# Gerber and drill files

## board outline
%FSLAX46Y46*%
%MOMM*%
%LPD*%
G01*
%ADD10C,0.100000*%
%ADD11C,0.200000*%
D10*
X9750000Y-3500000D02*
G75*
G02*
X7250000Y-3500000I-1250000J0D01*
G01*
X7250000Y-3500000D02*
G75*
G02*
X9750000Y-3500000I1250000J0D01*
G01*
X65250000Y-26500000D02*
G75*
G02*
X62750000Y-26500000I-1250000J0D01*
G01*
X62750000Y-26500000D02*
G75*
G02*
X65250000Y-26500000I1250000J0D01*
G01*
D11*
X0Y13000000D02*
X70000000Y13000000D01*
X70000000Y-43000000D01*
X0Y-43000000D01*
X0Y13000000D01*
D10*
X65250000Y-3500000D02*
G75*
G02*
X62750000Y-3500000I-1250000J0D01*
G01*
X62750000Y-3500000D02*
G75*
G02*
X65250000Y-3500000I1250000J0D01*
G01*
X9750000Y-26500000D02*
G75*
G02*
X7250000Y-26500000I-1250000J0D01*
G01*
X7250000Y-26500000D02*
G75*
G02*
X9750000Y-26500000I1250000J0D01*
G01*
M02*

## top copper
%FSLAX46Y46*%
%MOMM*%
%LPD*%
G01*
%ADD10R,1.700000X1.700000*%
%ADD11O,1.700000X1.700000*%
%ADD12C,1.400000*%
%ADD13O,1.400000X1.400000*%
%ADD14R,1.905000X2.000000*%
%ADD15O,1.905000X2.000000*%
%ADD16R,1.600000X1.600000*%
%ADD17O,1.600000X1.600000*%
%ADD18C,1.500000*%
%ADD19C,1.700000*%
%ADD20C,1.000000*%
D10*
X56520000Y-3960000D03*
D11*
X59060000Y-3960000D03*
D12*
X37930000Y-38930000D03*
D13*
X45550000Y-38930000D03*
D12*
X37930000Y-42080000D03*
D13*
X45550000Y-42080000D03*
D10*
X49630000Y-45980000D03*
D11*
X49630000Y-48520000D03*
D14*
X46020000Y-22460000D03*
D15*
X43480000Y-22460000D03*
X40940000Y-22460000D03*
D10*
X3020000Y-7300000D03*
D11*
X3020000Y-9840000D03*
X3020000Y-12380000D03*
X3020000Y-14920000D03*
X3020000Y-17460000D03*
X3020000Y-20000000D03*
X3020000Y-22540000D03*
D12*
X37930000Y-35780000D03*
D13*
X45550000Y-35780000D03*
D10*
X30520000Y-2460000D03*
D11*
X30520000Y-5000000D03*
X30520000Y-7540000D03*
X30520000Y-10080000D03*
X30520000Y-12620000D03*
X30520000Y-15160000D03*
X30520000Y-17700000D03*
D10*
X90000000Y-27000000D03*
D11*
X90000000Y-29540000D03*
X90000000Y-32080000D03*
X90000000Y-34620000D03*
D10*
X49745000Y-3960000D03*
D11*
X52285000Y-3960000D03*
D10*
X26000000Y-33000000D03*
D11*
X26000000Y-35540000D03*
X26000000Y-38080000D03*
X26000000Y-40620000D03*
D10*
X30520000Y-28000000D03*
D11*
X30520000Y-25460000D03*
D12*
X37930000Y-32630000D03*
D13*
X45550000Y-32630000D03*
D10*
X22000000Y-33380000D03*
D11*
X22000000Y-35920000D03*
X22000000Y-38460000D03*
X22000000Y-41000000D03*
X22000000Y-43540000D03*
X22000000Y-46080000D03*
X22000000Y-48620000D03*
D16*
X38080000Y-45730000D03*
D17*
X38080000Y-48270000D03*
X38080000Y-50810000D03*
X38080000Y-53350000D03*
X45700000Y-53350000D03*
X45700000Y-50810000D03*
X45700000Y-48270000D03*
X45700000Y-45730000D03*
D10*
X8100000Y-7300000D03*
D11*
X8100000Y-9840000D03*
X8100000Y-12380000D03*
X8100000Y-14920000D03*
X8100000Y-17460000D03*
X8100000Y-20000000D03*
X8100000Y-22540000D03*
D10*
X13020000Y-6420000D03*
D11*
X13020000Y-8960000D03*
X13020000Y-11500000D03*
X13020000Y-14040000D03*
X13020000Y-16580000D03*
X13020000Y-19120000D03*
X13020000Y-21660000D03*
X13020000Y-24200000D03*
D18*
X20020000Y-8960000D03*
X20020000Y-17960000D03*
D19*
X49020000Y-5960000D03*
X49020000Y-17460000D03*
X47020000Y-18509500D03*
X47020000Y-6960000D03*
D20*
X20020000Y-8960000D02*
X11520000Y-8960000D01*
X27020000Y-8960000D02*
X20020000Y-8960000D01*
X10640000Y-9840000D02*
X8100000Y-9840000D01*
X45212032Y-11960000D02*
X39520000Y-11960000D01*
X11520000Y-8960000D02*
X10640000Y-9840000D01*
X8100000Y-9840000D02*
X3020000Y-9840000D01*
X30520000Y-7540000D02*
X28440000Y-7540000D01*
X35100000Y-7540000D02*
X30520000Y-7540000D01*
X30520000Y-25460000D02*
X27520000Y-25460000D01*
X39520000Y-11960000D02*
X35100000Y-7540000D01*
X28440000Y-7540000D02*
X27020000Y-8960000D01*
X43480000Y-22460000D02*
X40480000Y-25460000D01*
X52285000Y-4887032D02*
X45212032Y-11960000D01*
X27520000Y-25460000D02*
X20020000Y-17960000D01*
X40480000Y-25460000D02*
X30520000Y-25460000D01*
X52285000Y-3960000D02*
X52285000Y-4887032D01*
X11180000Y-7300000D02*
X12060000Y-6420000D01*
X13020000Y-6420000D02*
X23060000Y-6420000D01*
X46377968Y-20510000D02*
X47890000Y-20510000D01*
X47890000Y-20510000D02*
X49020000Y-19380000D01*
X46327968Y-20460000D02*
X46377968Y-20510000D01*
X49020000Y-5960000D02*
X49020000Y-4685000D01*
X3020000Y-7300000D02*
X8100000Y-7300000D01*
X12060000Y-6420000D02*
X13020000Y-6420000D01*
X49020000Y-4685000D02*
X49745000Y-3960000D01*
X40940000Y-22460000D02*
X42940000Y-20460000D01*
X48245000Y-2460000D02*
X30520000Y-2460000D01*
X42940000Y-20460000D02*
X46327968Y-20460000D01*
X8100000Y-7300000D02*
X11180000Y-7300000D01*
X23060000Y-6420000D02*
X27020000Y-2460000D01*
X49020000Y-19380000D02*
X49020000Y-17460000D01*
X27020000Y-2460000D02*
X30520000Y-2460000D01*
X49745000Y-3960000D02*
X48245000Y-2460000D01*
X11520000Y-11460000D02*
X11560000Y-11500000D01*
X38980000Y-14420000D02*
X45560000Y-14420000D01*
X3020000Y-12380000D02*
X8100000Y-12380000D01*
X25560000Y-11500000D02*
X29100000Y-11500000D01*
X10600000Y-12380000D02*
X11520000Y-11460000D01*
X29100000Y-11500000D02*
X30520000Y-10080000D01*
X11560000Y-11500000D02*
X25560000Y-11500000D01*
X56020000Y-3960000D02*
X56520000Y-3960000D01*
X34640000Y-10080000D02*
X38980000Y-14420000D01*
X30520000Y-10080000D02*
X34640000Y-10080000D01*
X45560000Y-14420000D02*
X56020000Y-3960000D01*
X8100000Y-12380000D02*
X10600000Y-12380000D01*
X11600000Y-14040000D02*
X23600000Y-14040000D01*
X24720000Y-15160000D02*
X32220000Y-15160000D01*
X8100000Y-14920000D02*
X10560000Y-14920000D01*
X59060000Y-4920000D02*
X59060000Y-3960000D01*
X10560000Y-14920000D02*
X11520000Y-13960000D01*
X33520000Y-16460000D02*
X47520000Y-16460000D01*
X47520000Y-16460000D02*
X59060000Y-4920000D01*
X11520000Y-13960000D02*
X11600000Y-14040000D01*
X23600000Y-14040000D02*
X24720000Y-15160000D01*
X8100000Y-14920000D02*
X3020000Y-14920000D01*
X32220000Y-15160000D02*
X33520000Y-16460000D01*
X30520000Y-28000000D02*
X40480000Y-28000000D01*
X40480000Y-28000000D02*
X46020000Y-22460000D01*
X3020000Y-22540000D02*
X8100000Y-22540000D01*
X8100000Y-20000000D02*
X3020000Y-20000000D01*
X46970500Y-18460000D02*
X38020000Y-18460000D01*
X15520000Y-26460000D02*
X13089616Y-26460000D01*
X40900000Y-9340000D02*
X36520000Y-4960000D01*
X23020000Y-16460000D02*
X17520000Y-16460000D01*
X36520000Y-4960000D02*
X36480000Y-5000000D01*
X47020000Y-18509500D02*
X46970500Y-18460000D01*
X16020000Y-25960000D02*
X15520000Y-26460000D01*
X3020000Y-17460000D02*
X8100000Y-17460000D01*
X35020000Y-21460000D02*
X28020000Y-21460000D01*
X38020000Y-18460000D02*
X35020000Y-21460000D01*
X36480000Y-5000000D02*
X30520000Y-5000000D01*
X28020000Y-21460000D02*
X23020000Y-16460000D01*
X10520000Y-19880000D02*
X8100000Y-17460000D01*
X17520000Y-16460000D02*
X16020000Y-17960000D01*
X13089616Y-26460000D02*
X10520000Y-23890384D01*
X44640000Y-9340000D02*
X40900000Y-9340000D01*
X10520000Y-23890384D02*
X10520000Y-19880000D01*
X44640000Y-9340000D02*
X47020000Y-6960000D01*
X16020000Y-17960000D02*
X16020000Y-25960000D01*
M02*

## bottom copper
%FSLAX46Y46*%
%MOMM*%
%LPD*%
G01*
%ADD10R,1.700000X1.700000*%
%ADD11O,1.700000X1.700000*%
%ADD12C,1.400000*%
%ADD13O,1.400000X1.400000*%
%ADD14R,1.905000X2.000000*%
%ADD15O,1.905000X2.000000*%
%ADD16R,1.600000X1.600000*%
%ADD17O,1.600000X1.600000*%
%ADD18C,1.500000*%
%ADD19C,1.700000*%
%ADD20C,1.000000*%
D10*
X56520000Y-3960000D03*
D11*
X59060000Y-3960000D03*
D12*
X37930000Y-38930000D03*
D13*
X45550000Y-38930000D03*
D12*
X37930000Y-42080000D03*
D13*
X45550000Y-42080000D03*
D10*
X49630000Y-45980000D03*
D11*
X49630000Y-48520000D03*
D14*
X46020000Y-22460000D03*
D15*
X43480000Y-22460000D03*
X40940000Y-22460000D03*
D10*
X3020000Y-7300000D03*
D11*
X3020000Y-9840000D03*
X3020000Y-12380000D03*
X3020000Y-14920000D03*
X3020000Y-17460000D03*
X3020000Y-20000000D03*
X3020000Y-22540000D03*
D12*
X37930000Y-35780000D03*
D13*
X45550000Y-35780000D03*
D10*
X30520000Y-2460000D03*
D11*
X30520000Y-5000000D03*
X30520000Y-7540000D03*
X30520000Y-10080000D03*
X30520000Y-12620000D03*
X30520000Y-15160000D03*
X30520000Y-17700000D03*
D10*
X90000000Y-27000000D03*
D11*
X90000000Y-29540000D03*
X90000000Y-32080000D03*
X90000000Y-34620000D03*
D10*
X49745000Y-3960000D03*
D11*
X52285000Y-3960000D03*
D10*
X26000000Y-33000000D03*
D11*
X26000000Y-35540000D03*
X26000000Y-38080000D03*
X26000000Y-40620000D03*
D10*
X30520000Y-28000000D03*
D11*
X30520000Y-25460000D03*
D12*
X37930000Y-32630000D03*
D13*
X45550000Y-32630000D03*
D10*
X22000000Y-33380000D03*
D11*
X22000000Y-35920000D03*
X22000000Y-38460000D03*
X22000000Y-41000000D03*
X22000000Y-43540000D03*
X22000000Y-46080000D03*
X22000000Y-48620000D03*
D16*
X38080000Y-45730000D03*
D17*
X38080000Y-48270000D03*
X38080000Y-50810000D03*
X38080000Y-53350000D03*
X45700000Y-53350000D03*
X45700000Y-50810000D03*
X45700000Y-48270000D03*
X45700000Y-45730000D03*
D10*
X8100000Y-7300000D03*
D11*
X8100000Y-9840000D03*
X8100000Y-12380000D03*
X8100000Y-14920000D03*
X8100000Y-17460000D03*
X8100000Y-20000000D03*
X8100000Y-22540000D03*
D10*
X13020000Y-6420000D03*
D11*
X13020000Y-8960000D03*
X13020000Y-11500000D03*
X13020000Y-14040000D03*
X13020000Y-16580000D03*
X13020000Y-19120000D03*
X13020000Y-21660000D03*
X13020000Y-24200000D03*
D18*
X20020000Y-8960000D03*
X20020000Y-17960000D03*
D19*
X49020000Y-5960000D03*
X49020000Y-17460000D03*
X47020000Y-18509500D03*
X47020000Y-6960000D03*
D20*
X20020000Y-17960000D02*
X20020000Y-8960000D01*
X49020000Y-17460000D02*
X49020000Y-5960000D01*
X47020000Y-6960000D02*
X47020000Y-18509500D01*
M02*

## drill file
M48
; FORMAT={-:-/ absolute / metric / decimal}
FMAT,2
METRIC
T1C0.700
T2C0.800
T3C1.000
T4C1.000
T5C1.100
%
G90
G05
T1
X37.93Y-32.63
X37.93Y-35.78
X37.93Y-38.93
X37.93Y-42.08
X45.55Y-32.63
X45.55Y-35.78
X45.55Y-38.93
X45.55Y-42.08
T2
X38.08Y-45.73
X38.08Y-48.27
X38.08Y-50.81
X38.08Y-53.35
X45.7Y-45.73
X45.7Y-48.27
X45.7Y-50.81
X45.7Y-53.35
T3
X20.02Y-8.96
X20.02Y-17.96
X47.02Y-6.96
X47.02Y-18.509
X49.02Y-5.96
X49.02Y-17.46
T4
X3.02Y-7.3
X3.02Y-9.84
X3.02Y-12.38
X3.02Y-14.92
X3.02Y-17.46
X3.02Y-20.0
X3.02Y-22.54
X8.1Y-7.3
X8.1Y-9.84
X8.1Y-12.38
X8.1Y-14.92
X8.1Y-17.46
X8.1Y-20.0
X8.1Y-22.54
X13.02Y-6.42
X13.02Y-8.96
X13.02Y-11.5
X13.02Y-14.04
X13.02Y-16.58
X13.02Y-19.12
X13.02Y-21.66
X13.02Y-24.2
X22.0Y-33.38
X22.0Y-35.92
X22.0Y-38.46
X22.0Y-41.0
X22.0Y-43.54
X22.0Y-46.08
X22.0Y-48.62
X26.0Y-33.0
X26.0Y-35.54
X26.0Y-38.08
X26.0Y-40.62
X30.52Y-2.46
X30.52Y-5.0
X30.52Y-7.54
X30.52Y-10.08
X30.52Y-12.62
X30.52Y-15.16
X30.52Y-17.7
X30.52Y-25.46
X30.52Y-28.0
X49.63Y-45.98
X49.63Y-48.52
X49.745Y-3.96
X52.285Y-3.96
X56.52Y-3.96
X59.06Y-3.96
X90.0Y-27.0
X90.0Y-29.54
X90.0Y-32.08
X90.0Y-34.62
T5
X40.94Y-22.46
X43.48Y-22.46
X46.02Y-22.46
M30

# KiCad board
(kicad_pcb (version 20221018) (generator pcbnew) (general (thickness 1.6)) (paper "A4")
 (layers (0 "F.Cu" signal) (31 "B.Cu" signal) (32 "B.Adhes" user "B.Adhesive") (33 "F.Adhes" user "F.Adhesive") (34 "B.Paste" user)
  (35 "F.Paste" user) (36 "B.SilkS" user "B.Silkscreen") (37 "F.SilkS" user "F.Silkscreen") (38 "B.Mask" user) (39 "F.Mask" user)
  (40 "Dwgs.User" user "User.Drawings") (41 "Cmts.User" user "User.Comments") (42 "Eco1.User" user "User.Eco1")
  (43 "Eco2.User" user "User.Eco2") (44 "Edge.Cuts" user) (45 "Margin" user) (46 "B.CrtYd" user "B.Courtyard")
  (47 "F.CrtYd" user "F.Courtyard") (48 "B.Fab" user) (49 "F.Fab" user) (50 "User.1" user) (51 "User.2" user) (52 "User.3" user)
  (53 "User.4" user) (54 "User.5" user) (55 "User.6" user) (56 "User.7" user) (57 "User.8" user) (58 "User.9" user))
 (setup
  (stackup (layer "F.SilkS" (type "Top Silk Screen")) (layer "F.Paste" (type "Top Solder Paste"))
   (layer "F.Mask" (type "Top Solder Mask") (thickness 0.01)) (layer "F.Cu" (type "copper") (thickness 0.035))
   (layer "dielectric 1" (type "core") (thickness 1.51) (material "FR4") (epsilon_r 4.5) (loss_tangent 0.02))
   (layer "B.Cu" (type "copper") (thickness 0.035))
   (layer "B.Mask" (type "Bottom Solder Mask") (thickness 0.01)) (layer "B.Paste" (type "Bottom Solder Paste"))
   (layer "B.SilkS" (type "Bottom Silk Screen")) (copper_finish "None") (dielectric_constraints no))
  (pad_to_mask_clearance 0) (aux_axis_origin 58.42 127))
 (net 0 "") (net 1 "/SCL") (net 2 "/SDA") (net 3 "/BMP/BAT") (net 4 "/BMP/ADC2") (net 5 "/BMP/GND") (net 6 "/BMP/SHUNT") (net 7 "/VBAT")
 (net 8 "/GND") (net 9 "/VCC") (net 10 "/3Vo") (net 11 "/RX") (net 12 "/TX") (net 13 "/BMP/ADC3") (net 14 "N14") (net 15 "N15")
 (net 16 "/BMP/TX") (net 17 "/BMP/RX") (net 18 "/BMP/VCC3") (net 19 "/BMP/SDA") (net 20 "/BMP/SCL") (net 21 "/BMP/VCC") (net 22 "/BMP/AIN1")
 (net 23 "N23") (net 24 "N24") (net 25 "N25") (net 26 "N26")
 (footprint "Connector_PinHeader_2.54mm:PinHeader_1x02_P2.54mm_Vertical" (layer "F.Cu") (at 56.52 3.96 90)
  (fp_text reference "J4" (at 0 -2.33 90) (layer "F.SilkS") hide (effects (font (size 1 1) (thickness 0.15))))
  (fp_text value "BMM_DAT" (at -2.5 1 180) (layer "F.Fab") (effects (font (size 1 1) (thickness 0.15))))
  (pad "1" thru_hole rect (at 0 0 90) (size 1.7 1.7) (drill 1) (layers "*.Cu" "*.Mask") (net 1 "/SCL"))
  (pad "2" thru_hole oval (at 0 2.54 90) (size 1.7 1.7) (drill 1) (layers "*.Cu" "*.Mask") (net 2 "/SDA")))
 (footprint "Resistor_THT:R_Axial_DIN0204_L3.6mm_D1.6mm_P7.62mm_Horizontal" (layer "F.Cu") (at 37.93 38.93)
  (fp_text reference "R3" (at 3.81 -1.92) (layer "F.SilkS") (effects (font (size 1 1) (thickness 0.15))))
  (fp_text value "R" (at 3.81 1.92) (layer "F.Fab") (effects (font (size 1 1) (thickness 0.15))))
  (pad "1" thru_hole circle (at 0 0) (size 1.4 1.4) (drill 0.7) (layers "*.Cu" "*.Mask") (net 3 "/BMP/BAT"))
  (pad "2" thru_hole oval (at 7.62 0) (size 1.4 1.4) (drill 0.7) (layers "*.Cu" "*.Mask") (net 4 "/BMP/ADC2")))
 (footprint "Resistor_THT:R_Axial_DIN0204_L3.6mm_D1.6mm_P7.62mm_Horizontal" (layer "F.Cu") (at 37.93 42.08)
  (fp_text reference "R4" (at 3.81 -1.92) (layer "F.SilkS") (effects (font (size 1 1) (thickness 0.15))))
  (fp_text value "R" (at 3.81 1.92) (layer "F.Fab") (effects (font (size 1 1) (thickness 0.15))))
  (pad "1" thru_hole circle (at 0 0) (size 1.4 1.4) (drill 0.7) (layers "*.Cu" "*.Mask") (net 4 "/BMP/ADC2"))
  (pad "2" thru_hole oval (at 7.62 0) (size 1.4 1.4) (drill 0.7) (layers "*.Cu" "*.Mask") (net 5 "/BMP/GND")))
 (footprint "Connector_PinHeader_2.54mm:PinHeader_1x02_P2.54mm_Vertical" (layer "F.Cu") (at 49.63 45.98)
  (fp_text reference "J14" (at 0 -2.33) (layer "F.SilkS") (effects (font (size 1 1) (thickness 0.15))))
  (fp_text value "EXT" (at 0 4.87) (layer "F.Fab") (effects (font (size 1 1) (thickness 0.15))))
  (pad "1" thru_hole rect (at 0 0) (size 1.7 1.7) (drill 1) (layers "*.Cu" "*.Mask") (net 3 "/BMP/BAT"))
  (pad "2" thru_hole oval (at 0 2.54) (size 1.7 1.7) (drill 1) (layers "*.Cu" "*.Mask") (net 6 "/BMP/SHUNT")))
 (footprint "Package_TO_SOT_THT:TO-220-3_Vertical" (layer "F.Cu") (at 46.02 22.46 180)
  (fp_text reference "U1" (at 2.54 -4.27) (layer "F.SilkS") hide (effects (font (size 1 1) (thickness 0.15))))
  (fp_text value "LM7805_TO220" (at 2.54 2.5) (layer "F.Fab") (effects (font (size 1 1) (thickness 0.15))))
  (pad "1" thru_hole rect (at 0 0 180) (size 1.905 2) (drill 1.1) (layers "*.Cu" "*.Mask") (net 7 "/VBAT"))
  (pad "2" thru_hole oval (at 2.54 0 180) (size 1.905 2) (drill 1.1) (layers "*.Cu" "*.Mask") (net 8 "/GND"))
  (pad "3" thru_hole oval (at 5.08 0 180) (size 1.905 2) (drill 1.1) (layers "*.Cu" "*.Mask") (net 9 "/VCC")))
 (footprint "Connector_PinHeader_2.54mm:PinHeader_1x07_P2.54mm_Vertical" (layer "F.Cu") (at 3.02 7.3)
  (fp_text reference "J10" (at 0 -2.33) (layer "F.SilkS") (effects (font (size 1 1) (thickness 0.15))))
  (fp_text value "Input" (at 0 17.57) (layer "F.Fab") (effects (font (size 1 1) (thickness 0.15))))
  (pad "1" thru_hole rect (at 0 0) (size 1.7 1.7) (drill 1) (layers "*.Cu" "*.Mask") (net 9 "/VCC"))
  (pad "2" thru_hole oval (at 0 2.54) (size 1.7 1.7) (drill 1) (layers "*.Cu" "*.Mask") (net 8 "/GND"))
  (pad "3" thru_hole oval (at 0 5.08) (size 1.7 1.7) (drill 1) (layers "*.Cu" "*.Mask") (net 1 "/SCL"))
  (pad "4" thru_hole oval (at 0 7.62) (size 1.7 1.7) (drill 1) (layers "*.Cu" "*.Mask") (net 2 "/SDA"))
  (pad "5" thru_hole oval (at 0 10.16) (size 1.7 1.7) (drill 1) (layers "*.Cu" "*.Mask") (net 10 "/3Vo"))
  (pad "6" thru_hole oval (at 0 12.7) (size 1.7 1.7) (drill 1) (layers "*.Cu" "*.Mask") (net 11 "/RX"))
  (pad "7" thru_hole oval (at 0 15.24) (size 1.7 1.7) (drill 1) (layers "*.Cu" "*.Mask") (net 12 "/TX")))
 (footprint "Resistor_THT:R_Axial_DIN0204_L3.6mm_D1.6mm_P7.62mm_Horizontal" (layer "F.Cu") (at 37.93 35.78)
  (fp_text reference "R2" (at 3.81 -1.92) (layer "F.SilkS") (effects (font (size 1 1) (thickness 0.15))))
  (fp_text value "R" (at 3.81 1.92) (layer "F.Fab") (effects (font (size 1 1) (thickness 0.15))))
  (pad "1" thru_hole circle (at 0 0) (size 1.4 1.4) (drill 0.7) (layers "*.Cu" "*.Mask") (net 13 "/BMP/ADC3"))
  (pad "2" thru_hole oval (at 7.62 0) (size 1.4 1.4) (drill 0.7) (layers "*.Cu" "*.Mask") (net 5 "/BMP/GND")))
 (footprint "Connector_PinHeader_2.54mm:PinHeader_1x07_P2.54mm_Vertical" (layer "F.Cu") (at 30.52 2.46)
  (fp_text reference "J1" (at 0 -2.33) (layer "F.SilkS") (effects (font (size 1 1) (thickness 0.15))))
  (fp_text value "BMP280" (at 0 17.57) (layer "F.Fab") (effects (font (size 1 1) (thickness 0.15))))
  (pad "1" thru_hole rect (at 0 0) (size 1.7 1.7) (drill 1) (layers "*.Cu" "*.Mask") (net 9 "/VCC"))
  (pad "2" thru_hole oval (at 0 2.54) (size 1.7 1.7) (drill 1) (layers "*.Cu" "*.Mask") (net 10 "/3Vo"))
  (pad "3" thru_hole oval (at 0 5.08) (size 1.7 1.7) (drill 1) (layers "*.Cu" "*.Mask") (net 8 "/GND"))
  (pad "4" thru_hole oval (at 0 7.62) (size 1.7 1.7) (drill 1) (layers "*.Cu" "*.Mask") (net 1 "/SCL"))
  (pad "5" thru_hole oval (at 0 10.16) (size 1.7 1.7) (drill 1) (layers "*.Cu" "*.Mask") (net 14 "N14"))
  (pad "6" thru_hole oval (at 0 12.7) (size 1.7 1.7) (drill 1) (layers "*.Cu" "*.Mask") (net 2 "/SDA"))
  (pad "7" thru_hole oval (at 0 15.24) (size 1.7 1.7) (drill 1) (layers "*.Cu" "*.Mask") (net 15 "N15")))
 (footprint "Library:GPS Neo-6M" (layer "F.Cu") (at 90 27)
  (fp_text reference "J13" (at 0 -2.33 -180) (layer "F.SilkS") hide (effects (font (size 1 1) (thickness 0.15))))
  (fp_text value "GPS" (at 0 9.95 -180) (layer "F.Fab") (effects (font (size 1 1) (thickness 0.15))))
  (pad "1" thru_hole rect (at 0 0) (size 1.7 1.7) (drill 1) (layers "*.Cu" "*.Mask") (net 5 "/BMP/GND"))
  (pad "2" thru_hole oval (at 0 2.54) (size 1.7 1.7) (drill 1) (layers "*.Cu" "*.Mask") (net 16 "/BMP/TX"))
  (pad "3" thru_hole oval (at 0 5.08) (size 1.7 1.7) (drill 1) (layers "*.Cu" "*.Mask") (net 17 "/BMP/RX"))
  (pad "4" thru_hole oval (at 0 7.62) (size 1.7 1.7) (drill 1) (layers "*.Cu" "*.Mask") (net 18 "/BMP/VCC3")))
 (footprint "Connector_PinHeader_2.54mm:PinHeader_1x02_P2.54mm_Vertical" (layer "F.Cu") (at 49.745 3.96 90)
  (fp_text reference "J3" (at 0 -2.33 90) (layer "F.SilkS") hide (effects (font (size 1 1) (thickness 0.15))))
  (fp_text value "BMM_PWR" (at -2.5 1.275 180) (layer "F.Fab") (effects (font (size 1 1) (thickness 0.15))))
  (pad "1" thru_hole rect (at 0 0 90) (size 1.7 1.7) (drill 1) (layers "*.Cu" "*.Mask") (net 9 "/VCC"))
  (pad "2" thru_hole oval (at 0 2.54 90) (size 1.7 1.7) (drill 1) (layers "*.Cu" "*.Mask") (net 8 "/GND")))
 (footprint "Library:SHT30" (layer "F.Cu") (at 26 33)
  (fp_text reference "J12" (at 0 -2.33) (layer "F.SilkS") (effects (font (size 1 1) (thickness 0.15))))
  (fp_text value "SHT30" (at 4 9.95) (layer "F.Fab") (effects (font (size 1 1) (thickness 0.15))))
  (pad "1" thru_hole rect (at 0 0) (size 1.7 1.7) (drill 1) (layers "*.Cu" "*.Mask") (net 18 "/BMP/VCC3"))
  (pad "2" thru_hole oval (at 0 2.54) (size 1.7 1.7) (drill 1) (layers "*.Cu" "*.Mask") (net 5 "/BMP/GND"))
  (pad "3" thru_hole oval (at 0 5.08) (size 1.7 1.7) (drill 1) (layers "*.Cu" "*.Mask") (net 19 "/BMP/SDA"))
  (pad "4" thru_hole oval (at 0 7.62) (size 1.7 1.7) (drill 1) (layers "*.Cu" "*.Mask") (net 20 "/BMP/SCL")))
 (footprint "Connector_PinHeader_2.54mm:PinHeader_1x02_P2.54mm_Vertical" (layer "F.Cu") (at 30.52 28 180)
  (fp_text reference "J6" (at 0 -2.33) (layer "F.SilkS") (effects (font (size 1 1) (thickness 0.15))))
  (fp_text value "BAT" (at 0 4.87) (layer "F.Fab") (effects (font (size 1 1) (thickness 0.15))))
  (pad "1" thru_hole rect (at 0 0 180) (size 1.7 1.7) (drill 1) (layers "*.Cu" "*.Mask") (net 7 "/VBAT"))
  (pad "2" thru_hole oval (at 0 2.54 180) (size 1.7 1.7) (drill 1) (layers "*.Cu" "*.Mask") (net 8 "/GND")))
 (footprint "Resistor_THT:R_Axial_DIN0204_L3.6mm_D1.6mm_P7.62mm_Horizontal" (layer "F.Cu") (at 37.93 32.63)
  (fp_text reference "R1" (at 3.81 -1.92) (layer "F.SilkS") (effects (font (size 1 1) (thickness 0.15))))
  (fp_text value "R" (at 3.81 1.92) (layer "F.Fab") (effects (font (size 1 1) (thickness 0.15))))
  (pad "1" thru_hole circle (at 0 0) (size 1.4 1.4) (drill 0.7) (layers "*.Cu" "*.Mask") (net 6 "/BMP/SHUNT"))
  (pad "2" thru_hole oval (at 7.62 0) (size 1.4 1.4) (drill 0.7) (layers "*.Cu" "*.Mask") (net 13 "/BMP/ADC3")))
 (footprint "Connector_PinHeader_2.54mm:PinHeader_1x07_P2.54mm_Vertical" (layer "F.Cu") (at 22 33.38)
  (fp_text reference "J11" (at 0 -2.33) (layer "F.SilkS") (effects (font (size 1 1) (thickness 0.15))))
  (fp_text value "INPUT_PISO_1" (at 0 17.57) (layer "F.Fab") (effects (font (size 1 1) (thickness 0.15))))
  (pad "1" thru_hole rect (at 0 0) (size 1.7 1.7) (drill 1) (layers "*.Cu" "*.Mask") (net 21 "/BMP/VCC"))
  (pad "2" thru_hole oval (at 0 2.54) (size 1.7 1.7) (drill 1) (layers "*.Cu" "*.Mask") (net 5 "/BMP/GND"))
  (pad "3" thru_hole oval (at 0 5.08) (size 1.7 1.7) (drill 1) (layers "*.Cu" "*.Mask") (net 20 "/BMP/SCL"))
  (pad "4" thru_hole oval (at 0 7.62) (size 1.7 1.7) (drill 1) (layers "*.Cu" "*.Mask") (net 19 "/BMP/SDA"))
  (pad "5" thru_hole oval (at 0 10.16) (size 1.7 1.7) (drill 1) (layers "*.Cu" "*.Mask") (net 18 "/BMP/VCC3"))
  (pad "6" thru_hole oval (at 0 12.7) (size 1.7 1.7) (drill 1) (layers "*.Cu" "*.Mask") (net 17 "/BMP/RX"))
  (pad "7" thru_hole oval (at 0 15.24) (size 1.7 1.7) (drill 1) (layers "*.Cu" "*.Mask") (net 16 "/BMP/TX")))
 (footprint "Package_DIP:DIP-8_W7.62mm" (layer "F.Cu") (at 38.08 45.73)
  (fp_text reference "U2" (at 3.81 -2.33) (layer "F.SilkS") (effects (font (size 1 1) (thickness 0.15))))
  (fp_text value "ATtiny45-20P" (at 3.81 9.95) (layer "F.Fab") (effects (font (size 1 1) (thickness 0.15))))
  (pad "1" thru_hole rect (at 0 0) (size 1.6 1.6) (drill 0.8) (layers "*.Cu" "*.Mask") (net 18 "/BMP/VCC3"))
  (pad "2" thru_hole oval (at 0 2.54) (size 1.6 1.6) (drill 0.8) (layers "*.Cu" "*.Mask") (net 13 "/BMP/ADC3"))
  (pad "3" thru_hole oval (at 0 5.08) (size 1.6 1.6) (drill 0.8) (layers "*.Cu" "*.Mask") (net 4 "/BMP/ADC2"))
  (pad "4" thru_hole oval (at 0 7.62) (size 1.6 1.6) (drill 0.8) (layers "*.Cu" "*.Mask") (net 5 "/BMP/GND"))
  (pad "5" thru_hole oval (at 7.62 7.62) (size 1.6 1.6) (drill 0.8) (layers "*.Cu" "*.Mask") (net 19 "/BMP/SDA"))
  (pad "6" thru_hole oval (at 7.62 5.08) (size 1.6 1.6) (drill 0.8) (layers "*.Cu" "*.Mask") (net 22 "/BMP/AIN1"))
  (pad "7" thru_hole oval (at 7.62 2.54) (size 1.6 1.6) (drill 0.8) (layers "*.Cu" "*.Mask") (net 20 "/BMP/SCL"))
  (pad "8" thru_hole oval (at 7.62 0) (size 1.6 1.6) (drill 0.8) (layers "*.Cu" "*.Mask") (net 18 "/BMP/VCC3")))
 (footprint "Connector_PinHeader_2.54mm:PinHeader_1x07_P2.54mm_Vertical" (layer "F.Cu") (at 8.1 7.3)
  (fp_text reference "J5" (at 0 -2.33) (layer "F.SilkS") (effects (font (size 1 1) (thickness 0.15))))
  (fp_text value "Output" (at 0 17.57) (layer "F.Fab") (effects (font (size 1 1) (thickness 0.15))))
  (pad "1" thru_hole rect (at 0 0) (size 1.7 1.7) (drill 1) (layers "*.Cu" "*.Mask") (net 9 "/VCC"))
  (pad "2" thru_hole oval (at 0 2.54) (size 1.7 1.7) (drill 1) (layers "*.Cu" "*.Mask") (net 8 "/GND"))
  (pad "3" thru_hole oval (at 0 5.08) (size 1.7 1.7) (drill 1) (layers "*.Cu" "*.Mask") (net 1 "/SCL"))
  (pad "4" thru_hole oval (at 0 7.62) (size 1.7 1.7) (drill 1) (layers "*.Cu" "*.Mask") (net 2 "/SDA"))
  (pad "5" thru_hole oval (at 0 10.16) (size 1.7 1.7) (drill 1) (layers "*.Cu" "*.Mask") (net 10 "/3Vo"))
  (pad "6" thru_hole oval (at 0 12.7) (size 1.7 1.7) (drill 1) (layers "*.Cu" "*.Mask") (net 11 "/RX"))
  (pad "7" thru_hole oval (at 0 15.24) (size 1.7 1.7) (drill 1) (layers "*.Cu" "*.Mask") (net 12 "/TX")))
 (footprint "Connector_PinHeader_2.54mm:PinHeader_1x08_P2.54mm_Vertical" (layer "F.Cu") (at 13.02 6.42)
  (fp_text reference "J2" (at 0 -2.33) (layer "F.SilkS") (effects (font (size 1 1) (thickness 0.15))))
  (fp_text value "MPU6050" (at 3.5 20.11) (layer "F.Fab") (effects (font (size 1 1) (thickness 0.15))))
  (pad "1" thru_hole rect (at 0 0) (size 1.7 1.7) (drill 1) (layers "*.Cu" "*.Mask") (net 9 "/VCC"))
  (pad "2" thru_hole oval (at 0 2.54) (size 1.7 1.7) (drill 1) (layers "*.Cu" "*.Mask") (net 8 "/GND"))
  (pad "3" thru_hole oval (at 0 5.08) (size 1.7 1.7) (drill 1) (layers "*.Cu" "*.Mask") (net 1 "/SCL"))
  (pad "4" thru_hole oval (at 0 7.62) (size 1.7 1.7) (drill 1) (layers "*.Cu" "*.Mask") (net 2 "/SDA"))
  (pad "5" thru_hole oval (at 0 10.16) (size 1.7 1.7) (drill 1) (layers "*.Cu" "*.Mask") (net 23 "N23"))
  (pad "6" thru_hole oval (at 0 12.7) (size 1.7 1.7) (drill 1) (layers "*.Cu" "*.Mask") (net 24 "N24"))
  (pad "7" thru_hole oval (at 0 15.24) (size 1.7 1.7) (drill 1) (layers "*.Cu" "*.Mask") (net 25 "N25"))
  (pad "8" thru_hole oval (at 0 17.78) (size 1.7 1.7) (drill 1) (layers "*.Cu" "*.Mask") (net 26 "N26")))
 (gr_circle (center 8.5 3.5) (end 9.75 3.5) (stroke (width 0.1) (type default)) (fill none) (layer "Edge.Cuts"))
 (gr_circle (center 64 26.5) (end 65.25 26.5) (stroke (width 0.1) (type default)) (fill none) (layer "Edge.Cuts"))
 (gr_rect (start 0 -13) (end 70 43) (stroke (width 0.2) (type default)) (fill none) (layer "Edge.Cuts"))
 (gr_circle (center 64 3.5) (end 65.25 3.5) (stroke (width 0.1) (type default)) (fill none) (layer "Edge.Cuts"))
 (gr_circle (center 8.5 26.5) (end 9.75 26.5) (stroke (width 0.1) (type default)) (fill none) (layer "Edge.Cuts"))
 (segment (start 20.02 8.96) (end 11.52 8.96) (width 1) (layer "F.Cu") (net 8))
 (segment (start 27.02 8.96) (end 20.02 8.96) (width 1) (layer "F.Cu") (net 8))
 (segment (start 10.64 9.84) (end 8.1 9.84) (width 1) (layer "F.Cu") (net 8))
 (segment (start 45.212032 11.96) (end 39.52 11.96) (width 1) (layer "F.Cu") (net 8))
 (segment (start 11.52 8.96) (end 10.64 9.84) (width 1) (layer "F.Cu") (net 8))
 (segment (start 8.1 9.84) (end 3.02 9.84) (width 1) (layer "F.Cu") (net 8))
 (segment (start 30.52 7.54) (end 28.44 7.54) (width 1) (layer "F.Cu") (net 8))
 (segment (start 35.1 7.54) (end 30.52 7.54) (width 1) (layer "F.Cu") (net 8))
 (segment (start 30.52 25.46) (end 27.52 25.46) (width 1) (layer "F.Cu") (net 8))
 (segment (start 39.52 11.96) (end 35.1 7.54) (width 1) (layer "F.Cu") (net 8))
 (segment (start 28.44 7.54) (end 27.02 8.96) (width 1) (layer "F.Cu") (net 8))
 (segment (start 43.48 22.46) (end 40.48 25.46) (width 1) (layer "F.Cu") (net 8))
 (segment (start 52.285 4.887032) (end 45.212032 11.96) (width 1) (layer "F.Cu") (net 8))
 (segment (start 27.52 25.46) (end 20.02 17.96) (width 1) (layer "F.Cu") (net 8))
 (segment (start 40.48 25.46) (end 30.52 25.46) (width 1) (layer "F.Cu") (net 8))
 (segment (start 52.285 3.96) (end 52.285 4.887032) (width 1) (layer "F.Cu") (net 8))
 (via (at 20.02 8.96) (size 1.5) (drill 1) (layers "F.Cu" "B.Cu") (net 8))
 (via (at 20.02 17.96) (size 1.5) (drill 1) (layers "F.Cu" "B.Cu") (free) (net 8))
 (segment (start 20.02 17.96) (end 20.02 8.96) (width 1) (layer "B.Cu") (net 8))
 (segment (start 11.18 7.3) (end 12.06 6.42) (width 1) (layer "F.Cu") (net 9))
 (segment (start 13.02 6.42) (end 23.06 6.42) (width 1) (layer "F.Cu") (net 9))
 (segment (start 46.377968 20.51) (end 47.89 20.51) (width 1) (layer "F.Cu") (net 9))
 (segment (start 47.89 20.51) (end 49.02 19.38) (width 1) (layer "F.Cu") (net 9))
 (segment (start 46.327968 20.46) (end 46.377968 20.51) (width 1) (layer "F.Cu") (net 9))
 (segment (start 49.02 5.96) (end 49.02 4.685) (width 1) (layer "F.Cu") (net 9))
 (segment (start 3.02 7.3) (end 8.1 7.3) (width 1) (layer "F.Cu") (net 9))
 (segment (start 12.06 6.42) (end 13.02 6.42) (width 1) (layer "F.Cu") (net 9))
 (segment (start 49.02 4.685) (end 49.745 3.96) (width 1) (layer "F.Cu") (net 9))
 (segment (start 40.94 22.46) (end 42.94 20.46) (width 1) (layer "F.Cu") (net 9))
 (segment (start 48.245 2.46) (end 30.52 2.46) (width 1) (layer "F.Cu") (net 9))
 (segment (start 42.94 20.46) (end 46.327968 20.46) (width 1) (layer "F.Cu") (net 9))
 (segment (start 8.1 7.3) (end 11.18 7.3) (width 1) (layer "F.Cu") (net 9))
 (segment (start 23.06 6.42) (end 27.02 2.46) (width 1) (layer "F.Cu") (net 9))
 (segment (start 49.02 19.38) (end 49.02 17.46) (width 1) (layer "F.Cu") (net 9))
 (segment (start 27.02 2.46) (end 30.52 2.46) (width 1) (layer "F.Cu") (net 9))
 (segment (start 49.745 3.96) (end 48.245 2.46) (width 1) (layer "F.Cu") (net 9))
 (via (at 49.02 5.96) (size 1.7) (drill 1) (layers "F.Cu" "B.Cu") (free) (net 9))
 (via (at 49.02 17.46) (size 1.7) (drill 1) (layers "F.Cu" "B.Cu") (free) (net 9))
 (segment (start 49.02 17.46) (end 49.02 5.96) (width 1) (layer "B.Cu") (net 9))
 (segment (start 11.52 11.46) (end 11.56 11.5) (width 1) (layer "F.Cu") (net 1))
 (segment (start 38.98 14.42) (end 45.56 14.42) (width 1) (layer "F.Cu") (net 1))
 (segment (start 3.02 12.38) (end 8.1 12.38) (width 1) (layer "F.Cu") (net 1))
 (segment (start 25.56 11.5) (end 29.1 11.5) (width 1) (layer "F.Cu") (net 1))
 (segment (start 10.6 12.38) (end 11.52 11.46) (width 1) (layer "F.Cu") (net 1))
 (segment (start 29.1 11.5) (end 30.52 10.08) (width 1) (layer "F.Cu") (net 1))
 (segment (start 11.56 11.5) (end 25.56 11.5) (width 1) (layer "F.Cu") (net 1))
 (segment (start 56.02 3.96) (end 56.52 3.96) (width 1) (layer "F.Cu") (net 1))
 (segment (start 34.64 10.08) (end 38.98 14.42) (width 1) (layer "F.Cu") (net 1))
 (segment (start 30.52 10.08) (end 34.64 10.08) (width 1) (layer "F.Cu") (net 1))
 (segment (start 45.56 14.42) (end 56.02 3.96) (width 1) (layer "F.Cu") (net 1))
 (segment (start 8.1 12.38) (end 10.6 12.38) (width 1) (layer "F.Cu") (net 1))
 (segment (start 11.6 14.04) (end 23.6 14.04) (width 1) (layer "F.Cu") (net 2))
 (segment (start 24.72 15.16) (end 32.22 15.16) (width 1) (layer "F.Cu") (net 2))
 (segment (start 8.1 14.92) (end 10.56 14.92) (width 1) (layer "F.Cu") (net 2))
 (segment (start 59.06 4.92) (end 59.06 3.96) (width 1) (layer "F.Cu") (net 2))
 (segment (start 10.56 14.92) (end 11.52 13.96) (width 1) (layer "F.Cu") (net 2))
 (segment (start 33.52 16.46) (end 47.52 16.46) (width 1) (layer "F.Cu") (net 2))
 (segment (start 47.52 16.46) (end 59.06 4.92) (width 1) (layer "F.Cu") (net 2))
 (segment (start 11.52 13.96) (end 11.6 14.04) (width 1) (layer "F.Cu") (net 2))
 (segment (start 23.6 14.04) (end 24.72 15.16) (width 1) (layer "F.Cu") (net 2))
 (segment (start 8.1 14.92) (end 3.02 14.92) (width 1) (layer "F.Cu") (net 2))
 (segment (start 32.22 15.16) (end 33.52 16.46) (width 1) (layer "F.Cu") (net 2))
 (segment (start 30.52 28) (end 40.48 28) (width 1) (layer "F.Cu") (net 7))
 (segment (start 40.48 28) (end 46.02 22.46) (width 1) (layer "F.Cu") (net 7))
 (segment (start 3.02 22.54) (end 8.1 22.54) (width 1) (layer "F.Cu") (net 12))
 (segment (start 8.1 20) (end 3.02 20) (width 1) (layer "F.Cu") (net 11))
 (segment (start 46.9705 18.46) (end 38.02 18.46) (width 1) (layer "F.Cu") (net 10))
 (segment (start 15.52 26.46) (end 13.089616 26.46) (width 1) (layer "F.Cu") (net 10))
 (segment (start 40.9 9.34) (end 36.52 4.96) (width 1) (layer "F.Cu") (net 10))
 (segment (start 23.02 16.46) (end 17.52 16.46) (width 1) (layer "F.Cu") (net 10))
 (segment (start 36.52 4.96) (end 36.48 5) (width 1) (layer "F.Cu") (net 10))
 (segment (start 47.02 18.5095) (end 46.9705 18.46) (width 1) (layer "F.Cu") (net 10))
 (segment (start 16.02 25.96) (end 15.52 26.46) (width 1) (layer "F.Cu") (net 10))
 (segment (start 3.02 17.46) (end 8.1 17.46) (width 1) (layer "F.Cu") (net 10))
 (segment (start 35.02 21.46) (end 28.02 21.46) (width 1) (layer "F.Cu") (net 10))
 (segment (start 38.02 18.46) (end 35.02 21.46) (width 1) (layer "F.Cu") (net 10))
 (segment (start 36.48 5) (end 30.52 5) (width 1) (layer "F.Cu") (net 10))
 (segment (start 28.02 21.46) (end 23.02 16.46) (width 1) (layer "F.Cu") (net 10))
 (segment (start 10.52 19.88) (end 8.1 17.46) (width 1) (layer "F.Cu") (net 10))
 (segment (start 17.52 16.46) (end 16.02 17.96) (width 1) (layer "F.Cu") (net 10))
 (segment (start 13.089616 26.46) (end 10.52 23.890384) (width 1) (layer "F.Cu") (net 10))
 (segment (start 44.64 9.34) (end 40.9 9.34) (width 1) (layer "F.Cu") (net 10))
 (segment (start 10.52 23.890384) (end 10.52 19.88) (width 1) (layer "F.Cu") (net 10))
 (segment (start 44.64 9.34) (end 47.02 6.96) (width 1) (layer "F.Cu") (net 10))
 (segment (start 16.02 17.96) (end 16.02 25.96) (width 1) (layer "F.Cu") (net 10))
 (via (at 47.02 18.5095) (size 1.7) (drill 1) (layers "F.Cu" "B.Cu") (free) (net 10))
 (via (at 47.02 6.96) (size 1.7) (drill 1) (layers "F.Cu" "B.Cu") (free) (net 10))
 (segment (start 47.02 6.96) (end 47.02 18.5095) (width 1) (layer "B.Cu") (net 10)))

